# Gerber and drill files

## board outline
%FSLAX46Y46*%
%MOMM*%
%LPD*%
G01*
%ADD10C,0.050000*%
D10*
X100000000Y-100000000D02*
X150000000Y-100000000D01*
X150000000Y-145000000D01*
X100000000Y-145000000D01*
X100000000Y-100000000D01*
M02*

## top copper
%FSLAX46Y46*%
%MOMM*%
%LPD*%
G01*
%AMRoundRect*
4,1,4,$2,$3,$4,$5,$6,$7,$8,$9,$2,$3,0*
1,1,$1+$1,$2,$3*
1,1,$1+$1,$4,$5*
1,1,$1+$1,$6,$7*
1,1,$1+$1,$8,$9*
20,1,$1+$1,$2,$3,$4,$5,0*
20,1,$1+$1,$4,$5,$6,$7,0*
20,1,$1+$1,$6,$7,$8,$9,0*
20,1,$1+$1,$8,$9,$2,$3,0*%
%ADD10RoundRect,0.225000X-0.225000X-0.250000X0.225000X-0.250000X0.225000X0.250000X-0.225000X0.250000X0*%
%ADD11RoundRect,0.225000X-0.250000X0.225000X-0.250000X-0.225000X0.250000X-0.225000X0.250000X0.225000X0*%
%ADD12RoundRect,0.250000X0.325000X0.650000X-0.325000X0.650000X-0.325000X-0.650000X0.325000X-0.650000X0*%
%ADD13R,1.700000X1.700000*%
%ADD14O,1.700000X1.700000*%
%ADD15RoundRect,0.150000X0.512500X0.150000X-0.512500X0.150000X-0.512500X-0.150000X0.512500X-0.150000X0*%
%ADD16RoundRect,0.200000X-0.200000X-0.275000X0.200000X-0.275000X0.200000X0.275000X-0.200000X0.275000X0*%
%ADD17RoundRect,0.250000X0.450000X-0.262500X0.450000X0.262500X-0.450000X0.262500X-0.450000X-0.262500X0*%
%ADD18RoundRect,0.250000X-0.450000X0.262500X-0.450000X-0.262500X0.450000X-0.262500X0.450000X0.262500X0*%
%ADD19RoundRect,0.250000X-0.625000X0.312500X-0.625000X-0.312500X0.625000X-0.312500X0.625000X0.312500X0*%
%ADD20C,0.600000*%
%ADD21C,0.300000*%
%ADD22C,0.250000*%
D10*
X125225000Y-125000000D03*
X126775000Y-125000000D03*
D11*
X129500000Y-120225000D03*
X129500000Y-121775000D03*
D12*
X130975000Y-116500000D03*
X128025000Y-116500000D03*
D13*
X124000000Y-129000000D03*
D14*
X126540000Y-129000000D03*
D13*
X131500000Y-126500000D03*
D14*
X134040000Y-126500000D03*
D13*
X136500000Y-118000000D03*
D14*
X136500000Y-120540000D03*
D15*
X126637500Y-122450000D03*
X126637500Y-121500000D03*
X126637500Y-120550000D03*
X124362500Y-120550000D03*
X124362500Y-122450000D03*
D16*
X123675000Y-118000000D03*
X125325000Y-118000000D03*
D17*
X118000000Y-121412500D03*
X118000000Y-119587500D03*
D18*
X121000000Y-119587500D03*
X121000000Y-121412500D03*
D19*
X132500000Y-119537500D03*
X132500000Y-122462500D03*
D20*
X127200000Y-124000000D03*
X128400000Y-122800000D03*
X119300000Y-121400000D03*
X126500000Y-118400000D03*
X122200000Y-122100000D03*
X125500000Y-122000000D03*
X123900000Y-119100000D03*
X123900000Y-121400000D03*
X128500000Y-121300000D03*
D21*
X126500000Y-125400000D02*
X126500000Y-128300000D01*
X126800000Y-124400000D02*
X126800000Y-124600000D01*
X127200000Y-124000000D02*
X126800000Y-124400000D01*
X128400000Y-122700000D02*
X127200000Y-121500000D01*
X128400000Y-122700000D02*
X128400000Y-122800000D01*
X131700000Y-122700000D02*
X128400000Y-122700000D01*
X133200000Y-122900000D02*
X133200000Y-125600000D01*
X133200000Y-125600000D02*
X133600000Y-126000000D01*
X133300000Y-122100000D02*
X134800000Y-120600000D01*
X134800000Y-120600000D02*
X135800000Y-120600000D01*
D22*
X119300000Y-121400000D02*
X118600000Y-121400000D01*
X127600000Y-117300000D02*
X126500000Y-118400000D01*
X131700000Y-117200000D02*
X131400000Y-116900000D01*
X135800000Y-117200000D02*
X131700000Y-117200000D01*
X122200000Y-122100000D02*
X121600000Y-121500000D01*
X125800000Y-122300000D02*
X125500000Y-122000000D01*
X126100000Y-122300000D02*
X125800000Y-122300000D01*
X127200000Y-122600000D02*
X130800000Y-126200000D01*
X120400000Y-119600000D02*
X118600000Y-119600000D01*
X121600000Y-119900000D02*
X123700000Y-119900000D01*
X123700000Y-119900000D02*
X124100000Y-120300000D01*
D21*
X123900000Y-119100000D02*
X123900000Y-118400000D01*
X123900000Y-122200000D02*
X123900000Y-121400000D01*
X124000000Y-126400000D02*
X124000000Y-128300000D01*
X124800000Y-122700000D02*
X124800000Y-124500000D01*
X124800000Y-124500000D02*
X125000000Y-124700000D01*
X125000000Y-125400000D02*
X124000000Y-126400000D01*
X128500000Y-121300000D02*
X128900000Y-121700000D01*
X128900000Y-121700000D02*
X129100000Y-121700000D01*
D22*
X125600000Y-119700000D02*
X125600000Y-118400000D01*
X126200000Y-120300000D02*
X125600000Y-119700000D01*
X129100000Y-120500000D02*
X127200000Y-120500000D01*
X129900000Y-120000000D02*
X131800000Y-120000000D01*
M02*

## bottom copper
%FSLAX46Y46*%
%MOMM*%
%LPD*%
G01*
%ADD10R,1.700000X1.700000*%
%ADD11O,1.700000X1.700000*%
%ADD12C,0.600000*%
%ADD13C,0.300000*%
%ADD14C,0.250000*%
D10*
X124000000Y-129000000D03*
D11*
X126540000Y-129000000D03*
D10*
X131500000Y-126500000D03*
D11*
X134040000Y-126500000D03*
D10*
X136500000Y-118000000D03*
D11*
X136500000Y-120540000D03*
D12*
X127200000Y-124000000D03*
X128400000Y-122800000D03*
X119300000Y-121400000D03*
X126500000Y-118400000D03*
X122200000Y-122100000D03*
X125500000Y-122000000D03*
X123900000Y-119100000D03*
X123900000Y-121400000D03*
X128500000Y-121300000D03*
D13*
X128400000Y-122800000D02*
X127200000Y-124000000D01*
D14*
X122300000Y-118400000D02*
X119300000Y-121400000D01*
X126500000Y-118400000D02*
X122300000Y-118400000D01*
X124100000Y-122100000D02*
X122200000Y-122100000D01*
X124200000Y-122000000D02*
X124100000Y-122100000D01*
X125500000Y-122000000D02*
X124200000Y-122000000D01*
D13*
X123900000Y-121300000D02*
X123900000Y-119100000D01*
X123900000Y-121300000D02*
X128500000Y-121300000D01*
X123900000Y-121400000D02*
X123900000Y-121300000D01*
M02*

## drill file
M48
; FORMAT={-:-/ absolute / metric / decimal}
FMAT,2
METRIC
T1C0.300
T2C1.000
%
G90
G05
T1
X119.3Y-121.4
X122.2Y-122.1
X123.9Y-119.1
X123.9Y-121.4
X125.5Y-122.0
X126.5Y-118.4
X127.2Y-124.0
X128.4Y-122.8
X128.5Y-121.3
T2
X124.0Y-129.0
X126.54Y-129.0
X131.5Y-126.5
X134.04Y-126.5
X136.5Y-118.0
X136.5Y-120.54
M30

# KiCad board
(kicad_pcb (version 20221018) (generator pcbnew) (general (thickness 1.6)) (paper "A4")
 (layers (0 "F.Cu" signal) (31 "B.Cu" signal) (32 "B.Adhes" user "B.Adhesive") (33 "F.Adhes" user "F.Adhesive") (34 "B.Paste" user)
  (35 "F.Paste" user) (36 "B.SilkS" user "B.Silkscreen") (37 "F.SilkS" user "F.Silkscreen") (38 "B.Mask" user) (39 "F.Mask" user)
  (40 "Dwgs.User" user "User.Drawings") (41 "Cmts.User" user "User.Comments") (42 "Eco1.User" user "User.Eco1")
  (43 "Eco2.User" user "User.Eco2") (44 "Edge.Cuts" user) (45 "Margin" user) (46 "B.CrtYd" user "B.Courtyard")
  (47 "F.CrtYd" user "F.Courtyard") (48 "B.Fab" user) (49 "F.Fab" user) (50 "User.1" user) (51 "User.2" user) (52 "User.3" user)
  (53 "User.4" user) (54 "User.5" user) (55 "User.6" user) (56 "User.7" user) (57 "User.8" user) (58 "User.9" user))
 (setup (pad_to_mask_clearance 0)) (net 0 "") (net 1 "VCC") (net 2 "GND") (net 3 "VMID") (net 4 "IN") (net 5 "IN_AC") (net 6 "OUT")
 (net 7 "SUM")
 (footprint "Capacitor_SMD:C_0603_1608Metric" (layer "F.Cu") (at 126 125)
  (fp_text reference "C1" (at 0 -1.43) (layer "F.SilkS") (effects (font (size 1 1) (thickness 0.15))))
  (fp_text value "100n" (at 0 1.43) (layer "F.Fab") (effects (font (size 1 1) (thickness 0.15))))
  (pad "1" smd roundrect (at -0.775 0) (size 0.9 0.95) (layers "F.Cu" "F.Paste" "F.Mask") (roundrect_rratio 0.25) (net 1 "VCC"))
  (pad "2" smd roundrect (at 0.775 0) (size 0.9 0.95) (layers "F.Cu" "F.Paste" "F.Mask") (roundrect_rratio 0.25) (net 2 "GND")))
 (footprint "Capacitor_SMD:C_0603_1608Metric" (layer "F.Cu") (at 129.5 121 -90)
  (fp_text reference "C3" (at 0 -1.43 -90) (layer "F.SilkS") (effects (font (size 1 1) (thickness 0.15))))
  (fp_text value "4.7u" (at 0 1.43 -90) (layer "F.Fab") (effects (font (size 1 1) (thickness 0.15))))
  (pad "1" smd roundrect (at -0.775 0 270) (size 0.9 0.95) (layers "F.Cu" "F.Paste" "F.Mask") (roundrect_rratio 0.25) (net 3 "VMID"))
  (pad "2" smd roundrect (at 0.775 0 270) (size 0.9 0.95) (layers "F.Cu" "F.Paste" "F.Mask") (roundrect_rratio 0.25) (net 1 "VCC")))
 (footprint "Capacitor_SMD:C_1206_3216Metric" (layer "F.Cu") (at 129.5 116.5 180)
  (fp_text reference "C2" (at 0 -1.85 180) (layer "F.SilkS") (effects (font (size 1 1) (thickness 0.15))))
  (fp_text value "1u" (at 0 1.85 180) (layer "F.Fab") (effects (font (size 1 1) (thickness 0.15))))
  (pad "1" smd roundrect (at -1.475 0 180) (size 1.15 1.8) (layers "F.Cu" "F.Paste" "F.Mask") (roundrect_rratio 0.217391) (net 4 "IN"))
  (pad "2" smd roundrect (at 1.475 0 180) (size 1.15 1.8) (layers "F.Cu" "F.Paste" "F.Mask") (roundrect_rratio 0.217391) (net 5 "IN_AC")))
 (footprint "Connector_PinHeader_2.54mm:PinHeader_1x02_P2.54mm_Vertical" (layer "F.Cu") (at 124 129 90)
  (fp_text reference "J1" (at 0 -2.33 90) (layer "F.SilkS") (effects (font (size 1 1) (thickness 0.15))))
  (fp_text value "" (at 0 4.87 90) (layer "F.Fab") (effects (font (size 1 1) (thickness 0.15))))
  (pad "1" thru_hole rect (at 0 0 90) (size 1.7 1.7) (drill 1) (layers "*.Cu" "*.Mask") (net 1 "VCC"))
  (pad "2" thru_hole oval (at 0 2.54 90) (size 1.7 1.7) (drill 1) (layers "*.Cu" "*.Mask") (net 2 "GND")))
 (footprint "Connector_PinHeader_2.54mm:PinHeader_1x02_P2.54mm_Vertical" (layer "F.Cu") (at 131.5 126.5 90)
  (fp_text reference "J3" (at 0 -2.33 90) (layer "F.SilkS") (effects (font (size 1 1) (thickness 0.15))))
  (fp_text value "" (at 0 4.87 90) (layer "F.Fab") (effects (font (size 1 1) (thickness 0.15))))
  (pad "1" thru_hole rect (at 0 0 90) (size 1.7 1.7) (drill 1) (layers "*.Cu" "*.Mask") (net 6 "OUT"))
  (pad "2" thru_hole oval (at 0 2.54 90) (size 1.7 1.7) (drill 1) (layers "*.Cu" "*.Mask") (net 2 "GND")))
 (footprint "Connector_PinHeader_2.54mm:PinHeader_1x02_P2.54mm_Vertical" (layer "F.Cu") (at 136.5 118)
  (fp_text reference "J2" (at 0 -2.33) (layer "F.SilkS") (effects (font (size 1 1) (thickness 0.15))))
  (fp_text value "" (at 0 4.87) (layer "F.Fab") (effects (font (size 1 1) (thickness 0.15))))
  (pad "1" thru_hole rect (at 0 0) (size 1.7 1.7) (drill 1) (layers "*.Cu" "*.Mask") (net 4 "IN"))
  (pad "2" thru_hole oval (at 0 2.54) (size 1.7 1.7) (drill 1) (layers "*.Cu" "*.Mask") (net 2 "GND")))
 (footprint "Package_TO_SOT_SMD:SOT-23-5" (layer "F.Cu") (at 125.5 121.5 180)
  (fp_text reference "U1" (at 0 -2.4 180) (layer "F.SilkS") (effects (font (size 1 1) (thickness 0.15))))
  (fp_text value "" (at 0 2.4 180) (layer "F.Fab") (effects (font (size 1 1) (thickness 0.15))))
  (pad "1" smd roundrect (at -1.1375 -0.95 180) (size 1.325 0.6) (layers "F.Cu" "F.Paste" "F.Mask") (roundrect_rratio 0.25) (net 6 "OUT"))
  (pad "2" smd roundrect (at -1.1375 0 180) (size 1.325 0.6) (layers "F.Cu" "F.Paste" "F.Mask") (roundrect_rratio 0.25) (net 2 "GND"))
  (pad "3" smd roundrect (at -1.1375 0.95 180) (size 1.325 0.6) (layers "F.Cu" "F.Paste" "F.Mask") (roundrect_rratio 0.25) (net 3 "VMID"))
  (pad "4" smd roundrect (at 1.1375 0.95 180) (size 1.325 0.6) (layers "F.Cu" "F.Paste" "F.Mask") (roundrect_rratio 0.25) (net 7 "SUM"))
  (pad "5" smd roundrect (at 1.1375 -0.95 180) (size 1.325 0.6) (layers "F.Cu" "F.Paste" "F.Mask") (roundrect_rratio 0.25) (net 1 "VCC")))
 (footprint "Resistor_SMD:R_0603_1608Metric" (layer "F.Cu") (at 124.5 118)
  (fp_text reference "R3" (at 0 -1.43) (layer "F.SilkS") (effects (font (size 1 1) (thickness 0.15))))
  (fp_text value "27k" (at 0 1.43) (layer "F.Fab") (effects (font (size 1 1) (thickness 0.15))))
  (pad "1" smd roundrect (at -0.825 0) (size 0.8 0.95) (layers "F.Cu" "F.Paste" "F.Mask") (roundrect_rratio 0.25) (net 1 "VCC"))
  (pad "2" smd roundrect (at 0.825 0) (size 0.8 0.95) (layers "F.Cu" "F.Paste" "F.Mask") (roundrect_rratio 0.25) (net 3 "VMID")))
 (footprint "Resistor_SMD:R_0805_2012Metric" (layer "F.Cu") (at 118 120.5 90)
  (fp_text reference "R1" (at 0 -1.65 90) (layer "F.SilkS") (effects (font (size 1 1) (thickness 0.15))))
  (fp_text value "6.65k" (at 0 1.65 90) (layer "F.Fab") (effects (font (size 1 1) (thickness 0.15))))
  (pad "1" smd roundrect (at -0.9125 0 90) (size 1.025 1.4) (layers "F.Cu" "F.Paste" "F.Mask") (roundrect_rratio 0.243902) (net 5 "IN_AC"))
  (pad "2" smd roundrect (at 0.9125 0 90) (size 1.025 1.4) (layers "F.Cu" "F.Paste" "F.Mask") (roundrect_rratio 0.243902) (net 7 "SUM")))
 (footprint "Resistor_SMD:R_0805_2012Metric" (layer "F.Cu") (at 121 120.5 -90)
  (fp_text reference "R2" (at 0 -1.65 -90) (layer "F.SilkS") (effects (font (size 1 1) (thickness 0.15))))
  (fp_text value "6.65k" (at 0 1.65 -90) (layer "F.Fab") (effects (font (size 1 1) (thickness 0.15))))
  (pad "1" smd roundrect (at -0.9125 0 270) (size 1.025 1.4) (layers "F.Cu" "F.Paste" "F.Mask") (roundrect_rratio 0.243902) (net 7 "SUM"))
  (pad "2" smd roundrect (at 0.9125 0 270) (size 1.025 1.4) (layers "F.Cu" "F.Paste" "F.Mask") (roundrect_rratio 0.243902) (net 6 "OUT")))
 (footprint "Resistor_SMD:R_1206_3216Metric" (layer "F.Cu") (at 132.5 121 -90)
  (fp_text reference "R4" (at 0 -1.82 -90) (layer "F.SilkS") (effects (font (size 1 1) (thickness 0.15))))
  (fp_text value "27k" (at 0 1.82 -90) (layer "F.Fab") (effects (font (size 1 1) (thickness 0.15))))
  (pad "1" smd roundrect (at -1.4625 0 270) (size 1.125 1.75) (layers "F.Cu" "F.Paste" "F.Mask") (roundrect_rratio 0.222222) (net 3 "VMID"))
  (pad "2" smd roundrect (at 1.4625 0 270) (size 1.125 1.75) (layers "F.Cu" "F.Paste" "F.Mask") (roundrect_rratio 0.222222) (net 2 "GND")))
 (gr_rect (start 100 100) (end 150 145) (stroke (width 0.05) (type default)) (fill none) (layer "Edge.Cuts"))
 (segment (start 126.5 125.4) (end 126.5 128.3) (width 0.3) (layer "F.Cu") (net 2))
 (segment (start 126.8 124.4) (end 126.8 124.6) (width 0.3) (layer "F.Cu") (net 2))
 (segment (start 127.2 124) (end 126.8 124.4) (width 0.3) (layer "F.Cu") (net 2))
 (segment (start 128.4 122.7) (end 127.2 121.5) (width 0.3) (layer "F.Cu") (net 2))
 (segment (start 128.4 122.7) (end 128.4 122.8) (width 0.3) (layer "F.Cu") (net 2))
 (segment (start 131.7 122.7) (end 128.4 122.7) (width 0.3) (layer "F.Cu") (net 2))
 (segment (start 133.2 122.9) (end 133.2 125.6) (width 0.3) (layer "F.Cu") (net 2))
 (segment (start 133.2 125.6) (end 133.6 126) (width 0.3) (layer "F.Cu") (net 2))
 (segment (start 133.3 122.1) (end 134.8 120.6) (width 0.3) (layer "F.Cu") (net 2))
 (segment (start 134.8 120.6) (end 135.8 120.6) (width 0.3) (layer "F.Cu") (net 2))
 (via (at 127.2 124) (size 0.6) (drill 0.3) (layers "F.Cu" "B.Cu") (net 2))
 (via (at 128.4 122.8) (size 0.6) (drill 0.3) (layers "F.Cu" "B.Cu") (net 2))
 (segment (start 119.3 121.4) (end 118.6 121.4) (width 0.25) (layer "F.Cu") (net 5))
 (segment (start 127.6 117.3) (end 126.5 118.4) (width 0.25) (layer "F.Cu") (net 5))
 (segment (start 128.4 122.8) (end 127.2 124) (width 0.3) (layer "B.Cu") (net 2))
 (segment (start 131.7 117.2) (end 131.4 116.9) (width 0.25) (layer "F.Cu") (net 4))
 (segment (start 135.8 117.2) (end 131.7 117.2) (width 0.25) (layer "F.Cu") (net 4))
 (via (at 119.3 121.4) (size 0.6) (drill 0.3) (layers "F.Cu" "B.Cu") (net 5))
 (via (at 126.5 118.4) (size 0.6) (drill 0.3) (layers "F.Cu" "B.Cu") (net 5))
 (segment (start 122.2 122.1) (end 121.6 121.5) (width 0.25) (layer "F.Cu") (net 6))
 (segment (start 122.3 118.4) (end 119.3 121.4) (width 0.25) (layer "B.Cu") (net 5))
 (segment (start 125.8 122.3) (end 125.5 122) (width 0.25) (layer "F.Cu") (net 6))
 (segment (start 126.1 122.3) (end 125.8 122.3) (width 0.25) (layer "F.Cu") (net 6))
 (segment (start 126.5 118.4) (end 122.3 118.4) (width 0.25) (layer "B.Cu") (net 5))
 (segment (start 127.2 122.6) (end 130.8 126.2) (width 0.25) (layer "F.Cu") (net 6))
 (via (at 122.2 122.1) (size 0.6) (drill 0.3) (layers "F.Cu" "B.Cu") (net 6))
 (via (at 125.5 122) (size 0.6) (drill 0.3) (layers "F.Cu" "B.Cu") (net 6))
 (segment (start 120.4 119.6) (end 118.6 119.6) (width 0.25) (layer "F.Cu") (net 7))
 (segment (start 121.6 119.9) (end 123.7 119.9) (width 0.25) (layer "F.Cu") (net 7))
 (segment (start 123.7 119.9) (end 124.1 120.3) (width 0.25) (layer "F.Cu") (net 7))
 (segment (start 123.9 119.1) (end 123.9 118.4) (width 0.3) (layer "F.Cu") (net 1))
 (segment (start 123.9 122.2) (end 123.9 121.4) (width 0.3) (layer "F.Cu") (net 1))
 (segment (start 124 126.4) (end 124 128.3) (width 0.3) (layer "F.Cu") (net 1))
 (segment (start 124.1 122.1) (end 122.2 122.1) (width 0.25) (layer "B.Cu") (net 6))
 (segment (start 124.2 122) (end 124.1 122.1) (width 0.25) (layer "B.Cu") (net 6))
 (segment (start 124.8 122.7) (end 124.8 124.5) (width 0.3) (layer "F.Cu") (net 1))
 (segment (start 124.8 124.5) (end 125 124.7) (width 0.3) (layer "F.Cu") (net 1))
 (segment (start 125 125.4) (end 124 126.4) (width 0.3) (layer "F.Cu") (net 1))
 (segment (start 125.5 122) (end 124.2 122) (width 0.25) (layer "B.Cu") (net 6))
 (segment (start 128.5 121.3) (end 128.9 121.7) (width 0.3) (layer "F.Cu") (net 1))
 (segment (start 128.9 121.7) (end 129.1 121.7) (width 0.3) (layer "F.Cu") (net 1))
 (via (at 123.9 119.1) (size 0.6) (drill 0.3) (layers "F.Cu" "B.Cu") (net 1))
 (via (at 123.9 121.4) (size 0.6) (drill 0.3) (layers "F.Cu" "B.Cu") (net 1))
 (via (at 128.5 121.3) (size 0.6) (drill 0.3) (layers "F.Cu" "B.Cu") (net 1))
 (segment (start 123.9 121.3) (end 123.9 119.1) (width 0.3) (layer "B.Cu") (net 1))
 (segment (start 123.9 121.3) (end 128.5 121.3) (width 0.3) (layer "B.Cu") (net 1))
 (segment (start 123.9 121.4) (end 123.9 121.3) (width 0.3) (layer "B.Cu") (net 1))
 (segment (start 125.6 119.7) (end 125.6 118.4) (width 0.25) (layer "F.Cu") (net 3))
 (segment (start 126.2 120.3) (end 125.6 119.7) (width 0.25) (layer "F.Cu") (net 3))
 (segment (start 129.1 120.5) (end 127.2 120.5) (width 0.25) (layer "F.Cu") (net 3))
 (segment (start 129.9 120) (end 131.8 120) (width 0.25) (layer "F.Cu") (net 3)))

